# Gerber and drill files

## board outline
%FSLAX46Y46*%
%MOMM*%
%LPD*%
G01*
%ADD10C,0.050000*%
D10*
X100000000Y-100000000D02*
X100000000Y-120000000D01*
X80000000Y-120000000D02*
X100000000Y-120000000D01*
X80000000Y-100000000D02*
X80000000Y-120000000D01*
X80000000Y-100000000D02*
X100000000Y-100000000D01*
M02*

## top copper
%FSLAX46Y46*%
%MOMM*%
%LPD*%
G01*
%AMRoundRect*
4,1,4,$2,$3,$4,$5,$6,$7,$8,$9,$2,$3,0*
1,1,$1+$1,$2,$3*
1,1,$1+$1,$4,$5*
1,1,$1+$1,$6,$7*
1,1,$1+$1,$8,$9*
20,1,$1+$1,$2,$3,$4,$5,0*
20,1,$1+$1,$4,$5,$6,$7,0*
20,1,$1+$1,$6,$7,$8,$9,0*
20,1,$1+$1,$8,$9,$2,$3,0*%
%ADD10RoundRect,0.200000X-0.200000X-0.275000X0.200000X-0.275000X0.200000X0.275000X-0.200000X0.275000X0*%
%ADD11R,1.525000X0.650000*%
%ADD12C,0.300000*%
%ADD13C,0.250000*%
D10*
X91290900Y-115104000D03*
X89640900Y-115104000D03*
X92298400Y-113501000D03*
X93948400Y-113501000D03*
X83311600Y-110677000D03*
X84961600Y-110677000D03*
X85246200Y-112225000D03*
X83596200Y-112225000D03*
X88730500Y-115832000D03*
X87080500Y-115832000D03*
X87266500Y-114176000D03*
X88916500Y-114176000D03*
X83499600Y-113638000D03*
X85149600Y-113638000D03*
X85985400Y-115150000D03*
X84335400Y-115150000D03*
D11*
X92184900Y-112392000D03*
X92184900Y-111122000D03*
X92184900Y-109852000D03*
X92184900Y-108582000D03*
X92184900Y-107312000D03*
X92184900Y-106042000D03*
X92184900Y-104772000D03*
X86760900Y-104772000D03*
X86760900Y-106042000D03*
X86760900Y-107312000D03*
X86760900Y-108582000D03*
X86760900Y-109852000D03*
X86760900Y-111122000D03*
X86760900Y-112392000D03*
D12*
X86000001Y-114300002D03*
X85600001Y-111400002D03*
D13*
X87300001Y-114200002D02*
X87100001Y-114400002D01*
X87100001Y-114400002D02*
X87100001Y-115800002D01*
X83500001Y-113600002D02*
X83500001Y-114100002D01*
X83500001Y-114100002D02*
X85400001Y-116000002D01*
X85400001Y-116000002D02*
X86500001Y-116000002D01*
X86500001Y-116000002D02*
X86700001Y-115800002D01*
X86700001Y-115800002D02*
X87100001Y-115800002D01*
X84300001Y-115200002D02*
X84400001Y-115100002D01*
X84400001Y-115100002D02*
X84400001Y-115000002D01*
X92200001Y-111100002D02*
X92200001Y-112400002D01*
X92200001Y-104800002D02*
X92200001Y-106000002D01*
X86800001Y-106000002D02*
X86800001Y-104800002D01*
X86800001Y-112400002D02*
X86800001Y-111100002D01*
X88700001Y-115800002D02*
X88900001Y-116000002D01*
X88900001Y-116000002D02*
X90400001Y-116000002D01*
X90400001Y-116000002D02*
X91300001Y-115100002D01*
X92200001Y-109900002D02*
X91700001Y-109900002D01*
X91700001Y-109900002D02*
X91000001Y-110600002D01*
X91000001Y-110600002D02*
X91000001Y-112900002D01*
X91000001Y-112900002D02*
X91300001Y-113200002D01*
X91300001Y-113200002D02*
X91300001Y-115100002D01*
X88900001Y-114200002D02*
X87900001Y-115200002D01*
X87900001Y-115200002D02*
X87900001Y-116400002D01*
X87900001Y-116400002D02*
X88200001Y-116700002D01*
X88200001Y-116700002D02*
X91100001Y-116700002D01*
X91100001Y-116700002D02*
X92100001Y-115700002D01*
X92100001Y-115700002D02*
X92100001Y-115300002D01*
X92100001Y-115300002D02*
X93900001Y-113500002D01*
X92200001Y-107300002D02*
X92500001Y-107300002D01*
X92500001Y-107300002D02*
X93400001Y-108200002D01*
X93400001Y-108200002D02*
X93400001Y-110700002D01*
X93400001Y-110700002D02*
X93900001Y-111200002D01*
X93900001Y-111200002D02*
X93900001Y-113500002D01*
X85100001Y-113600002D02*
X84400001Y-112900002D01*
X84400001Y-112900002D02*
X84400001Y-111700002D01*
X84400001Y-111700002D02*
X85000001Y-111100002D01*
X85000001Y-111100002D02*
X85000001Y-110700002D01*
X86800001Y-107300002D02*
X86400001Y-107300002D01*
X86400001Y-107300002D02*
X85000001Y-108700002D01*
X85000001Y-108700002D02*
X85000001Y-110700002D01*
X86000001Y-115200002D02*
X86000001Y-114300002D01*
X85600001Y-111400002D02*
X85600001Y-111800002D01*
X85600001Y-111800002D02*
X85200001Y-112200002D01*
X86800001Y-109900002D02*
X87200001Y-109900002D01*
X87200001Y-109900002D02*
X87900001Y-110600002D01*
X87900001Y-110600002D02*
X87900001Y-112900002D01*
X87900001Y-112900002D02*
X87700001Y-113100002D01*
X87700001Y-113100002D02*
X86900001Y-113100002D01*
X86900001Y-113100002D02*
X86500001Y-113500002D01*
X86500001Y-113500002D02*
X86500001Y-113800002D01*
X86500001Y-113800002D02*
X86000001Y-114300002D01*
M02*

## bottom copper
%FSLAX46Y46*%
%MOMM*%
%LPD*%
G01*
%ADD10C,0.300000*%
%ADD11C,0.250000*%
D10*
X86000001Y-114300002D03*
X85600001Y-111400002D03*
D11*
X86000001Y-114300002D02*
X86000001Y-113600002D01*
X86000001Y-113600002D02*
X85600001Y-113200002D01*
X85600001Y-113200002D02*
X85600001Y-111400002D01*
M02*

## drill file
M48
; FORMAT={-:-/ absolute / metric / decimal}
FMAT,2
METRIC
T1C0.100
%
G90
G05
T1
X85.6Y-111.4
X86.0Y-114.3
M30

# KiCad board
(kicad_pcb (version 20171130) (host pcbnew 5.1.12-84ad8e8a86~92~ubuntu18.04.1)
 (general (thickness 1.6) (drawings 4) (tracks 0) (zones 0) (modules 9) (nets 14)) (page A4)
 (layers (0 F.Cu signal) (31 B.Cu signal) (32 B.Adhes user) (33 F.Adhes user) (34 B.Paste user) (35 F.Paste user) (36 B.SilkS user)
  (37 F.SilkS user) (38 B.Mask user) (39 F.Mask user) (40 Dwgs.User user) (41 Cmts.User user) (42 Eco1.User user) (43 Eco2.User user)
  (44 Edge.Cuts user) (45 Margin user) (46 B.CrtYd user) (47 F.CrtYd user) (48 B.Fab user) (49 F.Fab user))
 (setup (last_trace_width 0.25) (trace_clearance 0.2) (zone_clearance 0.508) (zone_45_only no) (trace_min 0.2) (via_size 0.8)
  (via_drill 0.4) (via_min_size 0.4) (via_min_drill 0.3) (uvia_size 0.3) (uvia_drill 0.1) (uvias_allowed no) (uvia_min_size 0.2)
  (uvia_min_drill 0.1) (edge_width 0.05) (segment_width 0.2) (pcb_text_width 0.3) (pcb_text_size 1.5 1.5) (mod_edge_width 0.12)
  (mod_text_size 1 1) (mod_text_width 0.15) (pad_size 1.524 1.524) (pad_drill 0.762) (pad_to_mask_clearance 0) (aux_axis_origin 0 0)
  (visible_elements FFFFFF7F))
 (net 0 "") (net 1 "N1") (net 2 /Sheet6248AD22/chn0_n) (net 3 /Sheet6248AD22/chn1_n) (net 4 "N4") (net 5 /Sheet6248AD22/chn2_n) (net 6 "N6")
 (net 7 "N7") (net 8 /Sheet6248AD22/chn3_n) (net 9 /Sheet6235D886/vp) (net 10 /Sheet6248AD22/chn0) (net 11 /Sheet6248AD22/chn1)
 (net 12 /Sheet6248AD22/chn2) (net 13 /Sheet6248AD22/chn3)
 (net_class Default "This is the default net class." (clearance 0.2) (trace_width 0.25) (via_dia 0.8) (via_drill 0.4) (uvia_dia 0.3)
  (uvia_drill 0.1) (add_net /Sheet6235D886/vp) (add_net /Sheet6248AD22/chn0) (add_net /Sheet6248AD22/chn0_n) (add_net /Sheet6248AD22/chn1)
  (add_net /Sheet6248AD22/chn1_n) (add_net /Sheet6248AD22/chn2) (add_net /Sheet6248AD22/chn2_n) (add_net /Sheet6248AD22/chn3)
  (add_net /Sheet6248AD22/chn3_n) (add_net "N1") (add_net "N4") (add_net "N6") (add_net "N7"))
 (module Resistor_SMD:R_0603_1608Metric (layer F.Cu) (at 90.465900 115.104000)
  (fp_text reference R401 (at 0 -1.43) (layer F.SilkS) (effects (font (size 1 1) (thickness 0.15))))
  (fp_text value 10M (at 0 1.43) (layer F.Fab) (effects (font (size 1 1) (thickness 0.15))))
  (pad 2 smd roundrect (at 0.825 0) (size 0.8 0.95) (layers F.Cu F.Mask F.Paste) (roundrect_rratio 0.25) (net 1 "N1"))
  (pad 1 smd roundrect (at -0.825 0) (size 0.8 0.95) (layers F.Cu F.Mask F.Paste) (roundrect_rratio 0.25) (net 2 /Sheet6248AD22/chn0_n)))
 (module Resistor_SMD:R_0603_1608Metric (layer F.Cu) (at 93.123400 113.501000)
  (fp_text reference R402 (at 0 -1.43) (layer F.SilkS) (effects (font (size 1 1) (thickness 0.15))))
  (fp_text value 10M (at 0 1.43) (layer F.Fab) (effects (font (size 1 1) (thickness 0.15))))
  (pad 1 smd roundrect (at -0.825 0) (size 0.8 0.95) (layers F.Cu F.Mask F.Paste) (roundrect_rratio 0.25) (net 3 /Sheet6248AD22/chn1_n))
  (pad 2 smd roundrect (at 0.825 0) (size 0.8 0.95) (layers F.Cu F.Mask F.Paste) (roundrect_rratio 0.25) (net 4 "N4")))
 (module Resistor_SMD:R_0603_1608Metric (layer F.Cu) (at 84.136600 110.677000)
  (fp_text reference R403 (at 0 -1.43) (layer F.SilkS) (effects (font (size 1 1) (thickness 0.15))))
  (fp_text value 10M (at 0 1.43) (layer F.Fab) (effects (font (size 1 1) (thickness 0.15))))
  (pad 1 smd roundrect (at -0.825 0) (size 0.8 0.95) (layers F.Cu F.Mask F.Paste) (roundrect_rratio 0.25) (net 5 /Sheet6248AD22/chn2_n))
  (pad 2 smd roundrect (at 0.825 0) (size 0.8 0.95) (layers F.Cu F.Mask F.Paste) (roundrect_rratio 0.25) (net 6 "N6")))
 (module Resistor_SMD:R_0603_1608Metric (layer F.Cu) (at 84.421200 112.225000)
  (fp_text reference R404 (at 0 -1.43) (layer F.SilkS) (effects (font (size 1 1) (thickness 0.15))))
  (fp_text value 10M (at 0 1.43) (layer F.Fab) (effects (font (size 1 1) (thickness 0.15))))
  (pad 2 smd roundrect (at 0.825 0) (size 0.8 0.95) (layers F.Cu F.Mask F.Paste) (roundrect_rratio 0.25) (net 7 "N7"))
  (pad 1 smd roundrect (at -0.825 0) (size 0.8 0.95) (layers F.Cu F.Mask F.Paste) (roundrect_rratio 0.25) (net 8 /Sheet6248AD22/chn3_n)))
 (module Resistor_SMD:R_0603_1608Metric (layer F.Cu) (at 87.905500 115.832000)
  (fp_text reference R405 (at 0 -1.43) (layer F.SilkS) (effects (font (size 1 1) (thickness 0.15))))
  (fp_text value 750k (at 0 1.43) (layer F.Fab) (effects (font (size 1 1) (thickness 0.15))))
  (pad 2 smd roundrect (at 0.825 0) (size 0.8 0.95) (layers F.Cu F.Mask F.Paste) (roundrect_rratio 0.25) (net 1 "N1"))
  (pad 1 smd roundrect (at -0.825 0) (size 0.8 0.95) (layers F.Cu F.Mask F.Paste) (roundrect_rratio 0.25) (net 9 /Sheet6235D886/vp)))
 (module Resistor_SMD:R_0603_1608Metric (layer F.Cu) (at 88.091500 114.176000)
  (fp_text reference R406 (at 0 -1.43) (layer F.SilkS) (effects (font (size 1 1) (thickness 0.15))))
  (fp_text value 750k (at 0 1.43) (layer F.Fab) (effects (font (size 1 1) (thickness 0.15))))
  (pad 1 smd roundrect (at -0.825 0) (size 0.8 0.95) (layers F.Cu F.Mask F.Paste) (roundrect_rratio 0.25) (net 9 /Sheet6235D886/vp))
  (pad 2 smd roundrect (at 0.825 0) (size 0.8 0.95) (layers F.Cu F.Mask F.Paste) (roundrect_rratio 0.25) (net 4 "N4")))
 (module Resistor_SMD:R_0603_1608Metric (layer F.Cu) (at 84.324600 113.638000)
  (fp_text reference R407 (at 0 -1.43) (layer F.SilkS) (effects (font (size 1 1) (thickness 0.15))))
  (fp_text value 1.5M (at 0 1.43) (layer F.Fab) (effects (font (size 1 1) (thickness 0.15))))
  (pad 1 smd roundrect (at -0.825 0) (size 0.8 0.95) (layers F.Cu F.Mask F.Paste) (roundrect_rratio 0.25) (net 9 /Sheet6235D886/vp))
  (pad 2 smd roundrect (at 0.825 0) (size 0.8 0.95) (layers F.Cu F.Mask F.Paste) (roundrect_rratio 0.25) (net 6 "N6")))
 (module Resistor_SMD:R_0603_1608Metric (layer F.Cu) (at 85.160400 115.150000)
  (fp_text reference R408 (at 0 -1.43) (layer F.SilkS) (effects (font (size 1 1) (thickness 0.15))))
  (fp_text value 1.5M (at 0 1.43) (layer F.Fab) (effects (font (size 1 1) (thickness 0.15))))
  (pad 2 smd roundrect (at 0.825 0) (size 0.8 0.95) (layers F.Cu F.Mask F.Paste) (roundrect_rratio 0.25) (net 7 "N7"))
  (pad 1 smd roundrect (at -0.825 0) (size 0.8 0.95) (layers F.Cu F.Mask F.Paste) (roundrect_rratio 0.25) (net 9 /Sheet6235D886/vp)))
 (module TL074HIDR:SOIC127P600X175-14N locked (layer F.Cu) (at 89.472900 108.582000 180.000000)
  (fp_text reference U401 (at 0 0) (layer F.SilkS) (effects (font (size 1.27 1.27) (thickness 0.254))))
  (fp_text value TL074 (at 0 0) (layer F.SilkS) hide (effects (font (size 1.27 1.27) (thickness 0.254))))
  (pad 1 smd rect (at -2.712 -3.81 270.000000) (size 0.65 1.525) (layers F.Cu F.Mask F.Paste) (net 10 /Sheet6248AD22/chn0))
  (pad 2 smd rect (at -2.712 -2.54 270.000000) (size 0.65 1.525) (layers F.Cu F.Mask F.Paste) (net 10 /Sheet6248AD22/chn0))
  (pad 3 smd rect (at -2.712 -1.27 270.000000) (size 0.65 1.525) (layers F.Cu F.Mask F.Paste) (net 1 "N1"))
  (pad 4 smd rect (at -2.712 0 270.000000) (size 0.65 1.525) (layers F.Cu F.Mask F.Paste))
  (pad 5 smd rect (at -2.712 1.27 270.000000) (size 0.65 1.525) (layers F.Cu F.Mask F.Paste) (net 4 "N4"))
  (pad 6 smd rect (at -2.712 2.54 270.000000) (size 0.65 1.525) (layers F.Cu F.Mask F.Paste) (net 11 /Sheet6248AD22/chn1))
  (pad 7 smd rect (at -2.712 3.81 270.000000) (size 0.65 1.525) (layers F.Cu F.Mask F.Paste) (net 11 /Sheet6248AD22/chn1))
  (pad 8 smd rect (at 2.712 3.81 270.000000) (size 0.65 1.525) (layers F.Cu F.Mask F.Paste) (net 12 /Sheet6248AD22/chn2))
  (pad 9 smd rect (at 2.712 2.54 270.000000) (size 0.65 1.525) (layers F.Cu F.Mask F.Paste) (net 12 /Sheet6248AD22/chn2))
  (pad 10 smd rect (at 2.712 1.27 270.000000) (size 0.65 1.525) (layers F.Cu F.Mask F.Paste) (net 6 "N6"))
  (pad 11 smd rect (at 2.712 0 270.000000) (size 0.65 1.525) (layers F.Cu F.Mask F.Paste))
  (pad 12 smd rect (at 2.712 -1.27 270.000000) (size 0.65 1.525) (layers F.Cu F.Mask F.Paste) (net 7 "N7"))
  (pad 13 smd rect (at 2.712 -2.54 270.000000) (size 0.65 1.525) (layers F.Cu F.Mask F.Paste) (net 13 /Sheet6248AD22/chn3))
  (pad 14 smd rect (at 2.712 -3.81 270.000000) (size 0.65 1.525) (layers F.Cu F.Mask F.Paste) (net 13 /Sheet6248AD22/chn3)))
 (gr_line (start 100 100) (end 100 120) (layer Edge.Cuts) (width 0.05))
 (gr_line (start 80 120) (end 100 120) (layer Edge.Cuts) (width 0.05))
 (gr_line (start 80 100) (end 80 120) (layer Edge.Cuts) (width 0.05))
 (gr_line (start 80 100) (end 100 100) (layer Edge.Cuts) (width 0.05))
 (segment (start 87.300001 114.200002) (end 87.100001 114.400002) (width 0.250000) (layer F.Cu) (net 9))
 (segment (start 87.100001 114.400002) (end 87.100001 115.800002) (width 0.250000) (layer F.Cu) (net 9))
 (segment (start 83.500001 113.600002) (end 83.500001 114.100002) (width 0.250000) (layer F.Cu) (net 9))
 (segment (start 83.500001 114.100002) (end 85.400001 116.000002) (width 0.250000) (layer F.Cu) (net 9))
 (segment (start 85.400001 116.000002) (end 86.500001 116.000002) (width 0.250000) (layer F.Cu) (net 9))
 (segment (start 86.500001 116.000002) (end 86.700001 115.800002) (width 0.250000) (layer F.Cu) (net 9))
 (segment (start 86.700001 115.800002) (end 87.100001 115.800002) (width 0.250000) (layer F.Cu) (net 9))
 (segment (start 84.300001 115.200002) (end 84.400001 115.100002) (width 0.250000) (layer F.Cu) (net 9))
 (segment (start 84.400001 115.100002) (end 84.400001 115.000002) (width 0.250000) (layer F.Cu) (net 9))
 (segment (start 92.200001 111.100002) (end 92.200001 112.400002) (width 0.250000) (layer F.Cu) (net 10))
 (segment (start 92.200001 104.800002) (end 92.200001 106.000002) (width 0.250000) (layer F.Cu) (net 11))
 (segment (start 86.800001 106.000002) (end 86.800001 104.800002) (width 0.250000) (layer F.Cu) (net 12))
 (segment (start 86.800001 112.400002) (end 86.800001 111.100002) (width 0.250000) (layer F.Cu) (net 13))
 (segment (start 88.700001 115.800002) (end 88.900001 116.000002) (width 0.250000) (layer F.Cu) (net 1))
 (segment (start 88.900001 116.000002) (end 90.400001 116.000002) (width 0.250000) (layer F.Cu) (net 1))
 (segment (start 90.400001 116.000002) (end 91.300001 115.100002) (width 0.250000) (layer F.Cu) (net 1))
 (segment (start 92.200001 109.900002) (end 91.700001 109.900002) (width 0.250000) (layer F.Cu) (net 1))
 (segment (start 91.700001 109.900002) (end 91.000001 110.600002) (width 0.250000) (layer F.Cu) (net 1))
 (segment (start 91.000001 110.600002) (end 91.000001 112.900002) (width 0.250000) (layer F.Cu) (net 1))
 (segment (start 91.000001 112.900002) (end 91.300001 113.200002) (width 0.250000) (layer F.Cu) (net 1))
 (segment (start 91.300001 113.200002) (end 91.300001 115.100002) (width 0.250000) (layer F.Cu) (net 1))
 (segment (start 88.900001 114.200002) (end 87.900001 115.200002) (width 0.250000) (layer F.Cu) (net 4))
 (segment (start 87.900001 115.200002) (end 87.900001 116.400002) (width 0.250000) (layer F.Cu) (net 4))
 (segment (start 87.900001 116.400002) (end 88.200001 116.700002) (width 0.250000) (layer F.Cu) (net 4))
 (segment (start 88.200001 116.700002) (end 91.100001 116.700002) (width 0.250000) (layer F.Cu) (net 4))
 (segment (start 91.100001 116.700002) (end 92.100001 115.700002) (width 0.250000) (layer F.Cu) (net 4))
 (segment (start 92.100001 115.700002) (end 92.100001 115.300002) (width 0.250000) (layer F.Cu) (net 4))
 (segment (start 92.100001 115.300002) (end 93.900001 113.500002) (width 0.250000) (layer F.Cu) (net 4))
 (segment (start 92.200001 107.300002) (end 92.500001 107.300002) (width 0.250000) (layer F.Cu) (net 4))
 (segment (start 92.500001 107.300002) (end 93.400001 108.200002) (width 0.250000) (layer F.Cu) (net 4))
 (segment (start 93.400001 108.200002) (end 93.400001 110.700002) (width 0.250000) (layer F.Cu) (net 4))
 (segment (start 93.400001 110.700002) (end 93.900001 111.200002) (width 0.250000) (layer F.Cu) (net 4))
 (segment (start 93.900001 111.200002) (end 93.900001 113.500002) (width 0.250000) (layer F.Cu) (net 4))
 (segment (start 85.100001 113.600002) (end 84.400001 112.900002) (width 0.250000) (layer F.Cu) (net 6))
 (segment (start 84.400001 112.900002) (end 84.400001 111.700002) (width 0.250000) (layer F.Cu) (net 6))
 (segment (start 84.400001 111.700002) (end 85.000001 111.100002) (width 0.250000) (layer F.Cu) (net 6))
 (segment (start 85.000001 111.100002) (end 85.000001 110.700002) (width 0.250000) (layer F.Cu) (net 6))
 (segment (start 86.800001 107.300002) (end 86.400001 107.300002) (width 0.250000) (layer F.Cu) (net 6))
 (segment (start 86.400001 107.300002) (end 85.000001 108.700002) (width 0.250000) (layer F.Cu) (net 6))
 (segment (start 85.000001 108.700002) (end 85.000001 110.700002) (width 0.250000) (layer F.Cu) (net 6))
 (segment (start 86.000001 115.200002) (end 86.000001 114.300002) (width 0.250000) (layer F.Cu) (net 7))
 (segment (start 86.000001 114.300002) (end 86.000001 113.600002) (width 0.250000) (layer B.Cu) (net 7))
 (segment (start 86.000001 113.600002) (end 85.600001 113.200002) (width 0.250000) (layer B.Cu) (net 7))
 (segment (start 85.600001 113.200002) (end 85.600001 111.400002) (width 0.250000) (layer B.Cu) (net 7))
 (segment (start 85.600001 111.400002) (end 85.600001 111.800002) (width 0.250000) (layer F.Cu) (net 7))
 (segment (start 85.600001 111.800002) (end 85.200001 112.200002) (width 0.250000) (layer F.Cu) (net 7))
 (segment (start 86.800001 109.900002) (end 87.200001 109.900002) (width 0.250000) (layer F.Cu) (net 7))
 (segment (start 87.200001 109.900002) (end 87.900001 110.600002) (width 0.250000) (layer F.Cu) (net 7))
 (segment (start 87.900001 110.600002) (end 87.900001 112.900002) (width 0.250000) (layer F.Cu) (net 7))
 (segment (start 87.900001 112.900002) (end 87.700001 113.100002) (width 0.250000) (layer F.Cu) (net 7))
 (segment (start 87.700001 113.100002) (end 86.900001 113.100002) (width 0.250000) (layer F.Cu) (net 7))
 (segment (start 86.900001 113.100002) (end 86.500001 113.500002) (width 0.250000) (layer F.Cu) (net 7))
 (segment (start 86.500001 113.500002) (end 86.500001 113.800002) (width 0.250000) (layer F.Cu) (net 7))
 (segment (start 86.500001 113.800002) (end 86.000001 114.300002) (width 0.250000) (layer F.Cu) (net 7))
 (via micro (at 86.000001 114.300002) (size 0.300000) (drill 0.100000) (layers F.Cu B.Cu) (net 7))
 (via micro (at 85.600001 111.400002) (size 0.300000) (drill 0.100000) (layers F.Cu B.Cu) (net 7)))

